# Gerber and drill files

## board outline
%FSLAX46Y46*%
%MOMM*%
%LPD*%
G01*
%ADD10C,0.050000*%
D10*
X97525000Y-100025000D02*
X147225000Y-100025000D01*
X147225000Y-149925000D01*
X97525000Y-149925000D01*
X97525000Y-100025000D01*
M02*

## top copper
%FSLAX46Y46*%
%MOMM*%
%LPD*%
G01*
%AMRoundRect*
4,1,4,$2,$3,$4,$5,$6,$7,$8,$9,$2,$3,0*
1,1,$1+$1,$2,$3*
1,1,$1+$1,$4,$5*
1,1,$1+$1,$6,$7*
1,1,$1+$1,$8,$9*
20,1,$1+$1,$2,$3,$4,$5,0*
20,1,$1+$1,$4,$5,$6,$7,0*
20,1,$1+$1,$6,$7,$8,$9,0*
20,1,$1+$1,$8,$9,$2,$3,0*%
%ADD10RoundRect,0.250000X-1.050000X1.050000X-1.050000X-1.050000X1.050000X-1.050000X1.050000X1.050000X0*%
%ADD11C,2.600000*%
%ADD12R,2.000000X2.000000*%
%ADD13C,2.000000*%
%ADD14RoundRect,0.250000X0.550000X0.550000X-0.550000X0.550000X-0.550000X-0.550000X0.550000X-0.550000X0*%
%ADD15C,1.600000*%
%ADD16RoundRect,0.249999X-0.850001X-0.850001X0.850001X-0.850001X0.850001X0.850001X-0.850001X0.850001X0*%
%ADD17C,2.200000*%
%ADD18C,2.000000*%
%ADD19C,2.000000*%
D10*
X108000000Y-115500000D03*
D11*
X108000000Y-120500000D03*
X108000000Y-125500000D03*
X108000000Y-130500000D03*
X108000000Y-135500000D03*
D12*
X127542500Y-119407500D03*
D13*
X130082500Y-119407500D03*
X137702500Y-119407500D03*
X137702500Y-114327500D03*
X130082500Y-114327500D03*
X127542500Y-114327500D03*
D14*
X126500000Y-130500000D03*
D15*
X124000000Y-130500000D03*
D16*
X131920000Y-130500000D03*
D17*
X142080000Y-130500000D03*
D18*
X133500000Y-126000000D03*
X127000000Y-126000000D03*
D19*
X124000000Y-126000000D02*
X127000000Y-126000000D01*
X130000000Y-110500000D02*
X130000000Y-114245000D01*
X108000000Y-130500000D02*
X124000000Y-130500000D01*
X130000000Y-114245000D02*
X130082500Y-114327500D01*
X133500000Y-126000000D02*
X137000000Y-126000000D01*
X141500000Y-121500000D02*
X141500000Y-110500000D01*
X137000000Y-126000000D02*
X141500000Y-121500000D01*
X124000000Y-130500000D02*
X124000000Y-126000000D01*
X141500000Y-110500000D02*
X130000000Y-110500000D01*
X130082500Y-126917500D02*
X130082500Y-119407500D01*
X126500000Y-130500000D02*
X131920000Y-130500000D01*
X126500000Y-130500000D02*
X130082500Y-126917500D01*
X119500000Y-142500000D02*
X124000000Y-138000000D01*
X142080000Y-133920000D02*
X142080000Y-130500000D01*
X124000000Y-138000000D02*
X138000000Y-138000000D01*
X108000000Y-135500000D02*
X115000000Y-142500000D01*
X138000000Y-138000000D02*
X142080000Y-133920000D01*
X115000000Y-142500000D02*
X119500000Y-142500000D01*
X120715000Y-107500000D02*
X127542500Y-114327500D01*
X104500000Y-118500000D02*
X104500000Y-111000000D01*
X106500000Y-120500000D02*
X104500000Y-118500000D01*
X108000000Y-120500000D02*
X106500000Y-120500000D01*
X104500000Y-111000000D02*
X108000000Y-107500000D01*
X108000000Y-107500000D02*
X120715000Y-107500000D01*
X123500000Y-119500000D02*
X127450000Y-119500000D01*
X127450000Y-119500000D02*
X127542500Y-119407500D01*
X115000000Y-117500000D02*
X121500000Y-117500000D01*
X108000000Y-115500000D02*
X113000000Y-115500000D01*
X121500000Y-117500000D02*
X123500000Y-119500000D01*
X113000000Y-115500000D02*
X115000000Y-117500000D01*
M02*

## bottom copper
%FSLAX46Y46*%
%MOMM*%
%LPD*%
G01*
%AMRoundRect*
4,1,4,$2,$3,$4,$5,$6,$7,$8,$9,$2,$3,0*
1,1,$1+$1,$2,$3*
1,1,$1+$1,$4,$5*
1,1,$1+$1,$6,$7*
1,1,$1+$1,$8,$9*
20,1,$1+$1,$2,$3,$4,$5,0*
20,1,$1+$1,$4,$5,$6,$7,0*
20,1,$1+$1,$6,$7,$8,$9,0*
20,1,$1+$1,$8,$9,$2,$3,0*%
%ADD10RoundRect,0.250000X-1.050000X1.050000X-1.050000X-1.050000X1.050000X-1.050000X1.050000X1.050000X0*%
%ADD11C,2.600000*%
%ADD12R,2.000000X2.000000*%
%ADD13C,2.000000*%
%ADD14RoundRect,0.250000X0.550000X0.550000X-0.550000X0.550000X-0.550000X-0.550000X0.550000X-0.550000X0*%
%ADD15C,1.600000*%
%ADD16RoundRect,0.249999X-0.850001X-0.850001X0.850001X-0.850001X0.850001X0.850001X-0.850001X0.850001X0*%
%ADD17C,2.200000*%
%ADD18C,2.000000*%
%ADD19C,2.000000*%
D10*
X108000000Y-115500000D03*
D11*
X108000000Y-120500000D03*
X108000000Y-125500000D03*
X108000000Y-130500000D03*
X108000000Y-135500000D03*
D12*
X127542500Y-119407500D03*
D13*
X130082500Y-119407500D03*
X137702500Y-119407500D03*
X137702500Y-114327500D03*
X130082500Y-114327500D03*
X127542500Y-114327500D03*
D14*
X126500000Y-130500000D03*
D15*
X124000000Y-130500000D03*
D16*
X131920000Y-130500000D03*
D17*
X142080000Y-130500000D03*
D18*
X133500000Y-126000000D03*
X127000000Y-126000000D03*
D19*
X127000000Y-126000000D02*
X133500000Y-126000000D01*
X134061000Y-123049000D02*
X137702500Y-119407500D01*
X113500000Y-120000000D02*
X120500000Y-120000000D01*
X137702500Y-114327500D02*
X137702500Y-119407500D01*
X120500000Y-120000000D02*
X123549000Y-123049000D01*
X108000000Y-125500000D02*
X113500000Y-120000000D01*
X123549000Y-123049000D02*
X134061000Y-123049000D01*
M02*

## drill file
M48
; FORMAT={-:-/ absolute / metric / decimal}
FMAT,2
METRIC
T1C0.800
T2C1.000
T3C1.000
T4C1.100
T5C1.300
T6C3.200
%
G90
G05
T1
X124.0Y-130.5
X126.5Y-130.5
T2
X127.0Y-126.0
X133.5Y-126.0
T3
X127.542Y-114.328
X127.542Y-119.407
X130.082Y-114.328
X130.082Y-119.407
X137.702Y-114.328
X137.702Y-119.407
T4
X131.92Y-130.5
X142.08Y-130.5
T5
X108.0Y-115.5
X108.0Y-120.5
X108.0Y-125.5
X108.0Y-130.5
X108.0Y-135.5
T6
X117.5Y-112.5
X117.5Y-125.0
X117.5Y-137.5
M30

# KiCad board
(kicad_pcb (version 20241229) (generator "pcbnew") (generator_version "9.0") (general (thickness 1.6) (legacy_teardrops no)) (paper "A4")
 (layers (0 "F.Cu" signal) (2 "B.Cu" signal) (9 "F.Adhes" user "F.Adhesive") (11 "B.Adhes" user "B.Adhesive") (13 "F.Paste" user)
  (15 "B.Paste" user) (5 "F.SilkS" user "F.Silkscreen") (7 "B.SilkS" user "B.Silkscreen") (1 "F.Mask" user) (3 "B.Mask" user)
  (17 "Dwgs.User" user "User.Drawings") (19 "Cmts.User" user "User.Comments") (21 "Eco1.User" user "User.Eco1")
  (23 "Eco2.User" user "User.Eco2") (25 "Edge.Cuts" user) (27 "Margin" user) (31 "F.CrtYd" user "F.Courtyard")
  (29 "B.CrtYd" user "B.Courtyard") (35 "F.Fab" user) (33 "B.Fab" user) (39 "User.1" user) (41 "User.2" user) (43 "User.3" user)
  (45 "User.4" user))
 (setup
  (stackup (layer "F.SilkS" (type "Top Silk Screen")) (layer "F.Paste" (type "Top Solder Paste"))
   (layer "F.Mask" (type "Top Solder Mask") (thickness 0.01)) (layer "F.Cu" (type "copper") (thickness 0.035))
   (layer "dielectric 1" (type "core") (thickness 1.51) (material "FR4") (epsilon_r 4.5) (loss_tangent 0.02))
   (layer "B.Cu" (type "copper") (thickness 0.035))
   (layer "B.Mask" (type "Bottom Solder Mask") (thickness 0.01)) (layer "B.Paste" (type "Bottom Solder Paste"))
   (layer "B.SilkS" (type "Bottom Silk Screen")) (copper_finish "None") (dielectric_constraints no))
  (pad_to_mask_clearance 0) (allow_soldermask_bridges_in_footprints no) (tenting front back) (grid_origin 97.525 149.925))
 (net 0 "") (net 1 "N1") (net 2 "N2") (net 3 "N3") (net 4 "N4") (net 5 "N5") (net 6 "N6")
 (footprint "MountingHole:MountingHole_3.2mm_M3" (layer "F.Cu") (at 117.5 112.5 -90)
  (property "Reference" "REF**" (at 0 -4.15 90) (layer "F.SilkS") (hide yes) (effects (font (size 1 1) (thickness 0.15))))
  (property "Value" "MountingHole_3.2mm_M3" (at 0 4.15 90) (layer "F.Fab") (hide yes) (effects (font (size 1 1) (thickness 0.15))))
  (pad "" np_thru_hole circle (at 0 0 270) (size 3.2 3.2) (drill 3.2) (layers "*.Cu" "*.Mask")))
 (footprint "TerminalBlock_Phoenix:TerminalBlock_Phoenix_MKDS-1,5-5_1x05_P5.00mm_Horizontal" (layer "F.Cu") (at 108 115.5 -90)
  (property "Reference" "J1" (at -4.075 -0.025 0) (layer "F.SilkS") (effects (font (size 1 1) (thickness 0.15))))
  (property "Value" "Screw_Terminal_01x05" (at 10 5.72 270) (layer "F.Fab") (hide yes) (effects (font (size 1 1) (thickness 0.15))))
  (pad "1" thru_hole roundrect (at 0 0 270) (size 2.6 2.6) (drill 1.3) (layers "*.Cu" "*.Mask") (remove_unused_layers no)
   (roundrect_rratio 0.096154) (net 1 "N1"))
  (pad "2" thru_hole circle (at 5 0 270) (size 2.6 2.6) (drill 1.3) (layers "*.Cu" "*.Mask") (remove_unused_layers no) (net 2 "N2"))
  (pad "3" thru_hole circle (at 10 0 270) (size 2.6 2.6) (drill 1.3) (layers "*.Cu" "*.Mask") (remove_unused_layers no) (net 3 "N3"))
  (pad "4" thru_hole circle (at 15 0 270) (size 2.6 2.6) (drill 1.3) (layers "*.Cu" "*.Mask") (remove_unused_layers no) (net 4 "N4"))
  (pad "5" thru_hole circle (at 20 0 270) (size 2.6 2.6) (drill 1.3) (layers "*.Cu" "*.Mask") (remove_unused_layers no) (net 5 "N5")))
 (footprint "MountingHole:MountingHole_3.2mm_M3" (layer "F.Cu") (at 117.5 137.5 -90)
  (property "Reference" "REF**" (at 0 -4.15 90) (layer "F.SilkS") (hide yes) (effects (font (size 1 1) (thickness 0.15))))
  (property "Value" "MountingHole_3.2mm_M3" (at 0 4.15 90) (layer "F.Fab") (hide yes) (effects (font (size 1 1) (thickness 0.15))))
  (pad "" np_thru_hole circle (at 0 0 270) (size 3.2 3.2) (drill 3.2) (layers "*.Cu" "*.Mask")))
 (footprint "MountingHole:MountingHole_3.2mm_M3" (layer "F.Cu") (at 117.5 125 -90)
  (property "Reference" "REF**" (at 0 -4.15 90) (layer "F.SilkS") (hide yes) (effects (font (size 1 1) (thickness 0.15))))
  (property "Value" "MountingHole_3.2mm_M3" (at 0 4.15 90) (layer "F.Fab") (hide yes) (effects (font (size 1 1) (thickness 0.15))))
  (pad "" np_thru_hole circle (at 0 0 270) (size 3.2 3.2) (drill 3.2) (layers "*.Cu" "*.Mask")))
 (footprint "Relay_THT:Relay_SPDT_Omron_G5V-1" (layer "F.Cu") (at 127.5425 119.4075 90)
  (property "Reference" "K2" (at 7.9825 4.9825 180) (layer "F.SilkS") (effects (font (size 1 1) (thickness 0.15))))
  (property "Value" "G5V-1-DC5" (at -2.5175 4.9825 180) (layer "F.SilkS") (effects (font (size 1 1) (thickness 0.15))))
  (pad "1" thru_hole rect (at 0 0 90) (size 2 2) (drill 1) (layers "*.Cu" "*.Mask") (remove_unused_layers no) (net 1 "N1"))
  (pad "2" thru_hole circle (at 0 2.54 90) (size 2 2) (drill 1) (layers "*.Cu" "*.Mask") (remove_unused_layers no) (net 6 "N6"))
  (pad "5" thru_hole circle (at 0 10.16 90) (size 2 2) (drill 1) (layers "*.Cu" "*.Mask") (remove_unused_layers no) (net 3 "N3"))
  (pad "6" thru_hole circle (at 5.08 10.16 90) (size 2 2) (drill 1) (layers "*.Cu" "*.Mask") (remove_unused_layers no) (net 3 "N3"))
  (pad "9" thru_hole circle (at 5.08 2.54 90) (size 2 2) (drill 1) (layers "*.Cu" "*.Mask") (remove_unused_layers no) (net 4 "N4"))
  (pad "10" thru_hole circle (at 5.08 0 90) (size 2 2) (drill 1) (layers "*.Cu" "*.Mask") (remove_unused_layers no) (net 2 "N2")))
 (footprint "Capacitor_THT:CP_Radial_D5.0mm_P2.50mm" (layer "F.Cu") (at 126.5 130.5 180)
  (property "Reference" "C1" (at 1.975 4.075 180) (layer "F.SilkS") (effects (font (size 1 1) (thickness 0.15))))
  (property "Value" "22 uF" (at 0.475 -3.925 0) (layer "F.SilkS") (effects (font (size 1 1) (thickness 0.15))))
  (pad "1" thru_hole roundrect (at 0 0 180) (size 1.6 1.6) (drill 0.8) (layers "*.Cu" "*.Mask") (remove_unused_layers no)
   (roundrect_rratio 0.15625) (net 6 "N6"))
  (pad "2" thru_hole circle (at 2.5 0 180) (size 1.6 1.6) (drill 0.8) (layers "*.Cu" "*.Mask") (remove_unused_layers no) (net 4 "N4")))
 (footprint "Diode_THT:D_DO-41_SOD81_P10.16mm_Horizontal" (layer "F.Cu") (at 131.92 130.5)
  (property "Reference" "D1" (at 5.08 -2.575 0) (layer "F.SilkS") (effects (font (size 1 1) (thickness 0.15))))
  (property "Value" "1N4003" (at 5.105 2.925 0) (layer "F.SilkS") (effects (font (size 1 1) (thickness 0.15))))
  (pad "1" thru_hole roundrect (at 0 0) (size 2.2 2.2) (drill 1.1) (layers "*.Cu" "*.Mask") (remove_unused_layers no)
   (roundrect_rratio 0.113636) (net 6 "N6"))
  (pad "2" thru_hole circle (at 10.16 0) (size 2.2 2.2) (drill 1.1) (layers "*.Cu" "*.Mask") (remove_unused_layers no) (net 5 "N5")))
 (gr_rect (start 97.525 100.025) (end 147.225 149.925) (stroke (width 0.05) (type solid)) (fill no) (locked yes) (layer "Edge.Cuts"))
 (segment (start 124 126) (end 127 126) (width 2) (layer "F.Cu") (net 4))
 (segment (start 130 110.5) (end 130 114.245) (width 2) (layer "F.Cu") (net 4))
 (segment (start 108 130.5) (end 124 130.5) (width 2) (layer "F.Cu") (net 4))
 (segment (start 130 114.245) (end 130.0825 114.3275) (width 2) (layer "F.Cu") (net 4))
 (segment (start 133.5 126) (end 137 126) (width 2) (layer "F.Cu") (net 4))
 (segment (start 141.5 121.5) (end 141.5 110.5) (width 2) (layer "F.Cu") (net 4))
 (segment (start 137 126) (end 141.5 121.5) (width 2) (layer "F.Cu") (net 4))
 (segment (start 124 130.5) (end 124 126) (width 2) (layer "F.Cu") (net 4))
 (segment (start 141.5 110.5) (end 130 110.5) (width 2) (layer "F.Cu") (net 4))
 (via (at 133.5 126) (size 2) (drill 1) (layers "F.Cu" "B.Cu") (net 4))
 (via (at 127 126) (size 2) (drill 1) (layers "F.Cu" "B.Cu") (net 4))
 (segment (start 127 126) (end 133.5 126) (width 2) (layer "B.Cu") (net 4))
 (segment (start 130.0825 126.9175) (end 130.0825 119.4075) (width 2) (layer "F.Cu") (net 6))
 (segment (start 126.5 130.5) (end 131.92 130.5) (width 2) (layer "F.Cu") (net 6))
 (segment (start 126.5 130.5) (end 130.0825 126.9175) (width 2) (layer "F.Cu") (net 6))
 (segment (start 119.5 142.5) (end 124 138) (width 2) (layer "F.Cu") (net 5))
 (segment (start 142.08 133.92) (end 142.08 130.5) (width 2) (layer "F.Cu") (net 5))
 (segment (start 124 138) (end 138 138) (width 2) (layer "F.Cu") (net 5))
 (segment (start 108 135.5) (end 115 142.5) (width 2) (layer "F.Cu") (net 5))
 (segment (start 138 138) (end 142.08 133.92) (width 2) (layer "F.Cu") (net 5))
 (segment (start 115 142.5) (end 119.5 142.5) (width 2) (layer "F.Cu") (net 5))
 (segment (start 134.061 123.049) (end 137.7025 119.4075) (width 2) (layer "B.Cu") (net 3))
 (segment (start 113.5 120) (end 120.5 120) (width 2) (layer "B.Cu") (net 3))
 (segment (start 137.7025 114.3275) (end 137.7025 119.4075) (width 2) (layer "B.Cu") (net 3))
 (segment (start 120.5 120) (end 123.549 123.049) (width 2) (layer "B.Cu") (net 3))
 (segment (start 108 125.5) (end 113.5 120) (width 2) (layer "B.Cu") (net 3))
 (segment (start 123.549 123.049) (end 134.061 123.049) (width 2) (layer "B.Cu") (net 3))
 (segment (start 120.715 107.5) (end 127.5425 114.3275) (width 2) (layer "F.Cu") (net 2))
 (segment (start 104.5 118.5) (end 104.5 111) (width 2) (layer "F.Cu") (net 2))
 (segment (start 106.5 120.5) (end 104.5 118.5) (width 2) (layer "F.Cu") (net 2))
 (segment (start 108 120.5) (end 106.5 120.5) (width 2) (layer "F.Cu") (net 2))
 (segment (start 104.5 111) (end 108 107.5) (width 2) (layer "F.Cu") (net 2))
 (segment (start 108 107.5) (end 120.715 107.5) (width 2) (layer "F.Cu") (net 2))
 (segment (start 123.5 119.5) (end 127.45 119.5) (width 2) (layer "F.Cu") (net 1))
 (segment (start 127.45 119.5) (end 127.5425 119.4075) (width 2) (layer "F.Cu") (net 1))
 (segment (start 115 117.5) (end 121.5 117.5) (width 2) (layer "F.Cu") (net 1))
 (segment (start 108 115.5) (end 113 115.5) (width 2) (layer "F.Cu") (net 1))
 (segment (start 121.5 117.5) (end 123.5 119.5) (width 2) (layer "F.Cu") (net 1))
 (segment (start 113 115.5) (end 115 117.5) (width 2) (layer "F.Cu") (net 1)))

